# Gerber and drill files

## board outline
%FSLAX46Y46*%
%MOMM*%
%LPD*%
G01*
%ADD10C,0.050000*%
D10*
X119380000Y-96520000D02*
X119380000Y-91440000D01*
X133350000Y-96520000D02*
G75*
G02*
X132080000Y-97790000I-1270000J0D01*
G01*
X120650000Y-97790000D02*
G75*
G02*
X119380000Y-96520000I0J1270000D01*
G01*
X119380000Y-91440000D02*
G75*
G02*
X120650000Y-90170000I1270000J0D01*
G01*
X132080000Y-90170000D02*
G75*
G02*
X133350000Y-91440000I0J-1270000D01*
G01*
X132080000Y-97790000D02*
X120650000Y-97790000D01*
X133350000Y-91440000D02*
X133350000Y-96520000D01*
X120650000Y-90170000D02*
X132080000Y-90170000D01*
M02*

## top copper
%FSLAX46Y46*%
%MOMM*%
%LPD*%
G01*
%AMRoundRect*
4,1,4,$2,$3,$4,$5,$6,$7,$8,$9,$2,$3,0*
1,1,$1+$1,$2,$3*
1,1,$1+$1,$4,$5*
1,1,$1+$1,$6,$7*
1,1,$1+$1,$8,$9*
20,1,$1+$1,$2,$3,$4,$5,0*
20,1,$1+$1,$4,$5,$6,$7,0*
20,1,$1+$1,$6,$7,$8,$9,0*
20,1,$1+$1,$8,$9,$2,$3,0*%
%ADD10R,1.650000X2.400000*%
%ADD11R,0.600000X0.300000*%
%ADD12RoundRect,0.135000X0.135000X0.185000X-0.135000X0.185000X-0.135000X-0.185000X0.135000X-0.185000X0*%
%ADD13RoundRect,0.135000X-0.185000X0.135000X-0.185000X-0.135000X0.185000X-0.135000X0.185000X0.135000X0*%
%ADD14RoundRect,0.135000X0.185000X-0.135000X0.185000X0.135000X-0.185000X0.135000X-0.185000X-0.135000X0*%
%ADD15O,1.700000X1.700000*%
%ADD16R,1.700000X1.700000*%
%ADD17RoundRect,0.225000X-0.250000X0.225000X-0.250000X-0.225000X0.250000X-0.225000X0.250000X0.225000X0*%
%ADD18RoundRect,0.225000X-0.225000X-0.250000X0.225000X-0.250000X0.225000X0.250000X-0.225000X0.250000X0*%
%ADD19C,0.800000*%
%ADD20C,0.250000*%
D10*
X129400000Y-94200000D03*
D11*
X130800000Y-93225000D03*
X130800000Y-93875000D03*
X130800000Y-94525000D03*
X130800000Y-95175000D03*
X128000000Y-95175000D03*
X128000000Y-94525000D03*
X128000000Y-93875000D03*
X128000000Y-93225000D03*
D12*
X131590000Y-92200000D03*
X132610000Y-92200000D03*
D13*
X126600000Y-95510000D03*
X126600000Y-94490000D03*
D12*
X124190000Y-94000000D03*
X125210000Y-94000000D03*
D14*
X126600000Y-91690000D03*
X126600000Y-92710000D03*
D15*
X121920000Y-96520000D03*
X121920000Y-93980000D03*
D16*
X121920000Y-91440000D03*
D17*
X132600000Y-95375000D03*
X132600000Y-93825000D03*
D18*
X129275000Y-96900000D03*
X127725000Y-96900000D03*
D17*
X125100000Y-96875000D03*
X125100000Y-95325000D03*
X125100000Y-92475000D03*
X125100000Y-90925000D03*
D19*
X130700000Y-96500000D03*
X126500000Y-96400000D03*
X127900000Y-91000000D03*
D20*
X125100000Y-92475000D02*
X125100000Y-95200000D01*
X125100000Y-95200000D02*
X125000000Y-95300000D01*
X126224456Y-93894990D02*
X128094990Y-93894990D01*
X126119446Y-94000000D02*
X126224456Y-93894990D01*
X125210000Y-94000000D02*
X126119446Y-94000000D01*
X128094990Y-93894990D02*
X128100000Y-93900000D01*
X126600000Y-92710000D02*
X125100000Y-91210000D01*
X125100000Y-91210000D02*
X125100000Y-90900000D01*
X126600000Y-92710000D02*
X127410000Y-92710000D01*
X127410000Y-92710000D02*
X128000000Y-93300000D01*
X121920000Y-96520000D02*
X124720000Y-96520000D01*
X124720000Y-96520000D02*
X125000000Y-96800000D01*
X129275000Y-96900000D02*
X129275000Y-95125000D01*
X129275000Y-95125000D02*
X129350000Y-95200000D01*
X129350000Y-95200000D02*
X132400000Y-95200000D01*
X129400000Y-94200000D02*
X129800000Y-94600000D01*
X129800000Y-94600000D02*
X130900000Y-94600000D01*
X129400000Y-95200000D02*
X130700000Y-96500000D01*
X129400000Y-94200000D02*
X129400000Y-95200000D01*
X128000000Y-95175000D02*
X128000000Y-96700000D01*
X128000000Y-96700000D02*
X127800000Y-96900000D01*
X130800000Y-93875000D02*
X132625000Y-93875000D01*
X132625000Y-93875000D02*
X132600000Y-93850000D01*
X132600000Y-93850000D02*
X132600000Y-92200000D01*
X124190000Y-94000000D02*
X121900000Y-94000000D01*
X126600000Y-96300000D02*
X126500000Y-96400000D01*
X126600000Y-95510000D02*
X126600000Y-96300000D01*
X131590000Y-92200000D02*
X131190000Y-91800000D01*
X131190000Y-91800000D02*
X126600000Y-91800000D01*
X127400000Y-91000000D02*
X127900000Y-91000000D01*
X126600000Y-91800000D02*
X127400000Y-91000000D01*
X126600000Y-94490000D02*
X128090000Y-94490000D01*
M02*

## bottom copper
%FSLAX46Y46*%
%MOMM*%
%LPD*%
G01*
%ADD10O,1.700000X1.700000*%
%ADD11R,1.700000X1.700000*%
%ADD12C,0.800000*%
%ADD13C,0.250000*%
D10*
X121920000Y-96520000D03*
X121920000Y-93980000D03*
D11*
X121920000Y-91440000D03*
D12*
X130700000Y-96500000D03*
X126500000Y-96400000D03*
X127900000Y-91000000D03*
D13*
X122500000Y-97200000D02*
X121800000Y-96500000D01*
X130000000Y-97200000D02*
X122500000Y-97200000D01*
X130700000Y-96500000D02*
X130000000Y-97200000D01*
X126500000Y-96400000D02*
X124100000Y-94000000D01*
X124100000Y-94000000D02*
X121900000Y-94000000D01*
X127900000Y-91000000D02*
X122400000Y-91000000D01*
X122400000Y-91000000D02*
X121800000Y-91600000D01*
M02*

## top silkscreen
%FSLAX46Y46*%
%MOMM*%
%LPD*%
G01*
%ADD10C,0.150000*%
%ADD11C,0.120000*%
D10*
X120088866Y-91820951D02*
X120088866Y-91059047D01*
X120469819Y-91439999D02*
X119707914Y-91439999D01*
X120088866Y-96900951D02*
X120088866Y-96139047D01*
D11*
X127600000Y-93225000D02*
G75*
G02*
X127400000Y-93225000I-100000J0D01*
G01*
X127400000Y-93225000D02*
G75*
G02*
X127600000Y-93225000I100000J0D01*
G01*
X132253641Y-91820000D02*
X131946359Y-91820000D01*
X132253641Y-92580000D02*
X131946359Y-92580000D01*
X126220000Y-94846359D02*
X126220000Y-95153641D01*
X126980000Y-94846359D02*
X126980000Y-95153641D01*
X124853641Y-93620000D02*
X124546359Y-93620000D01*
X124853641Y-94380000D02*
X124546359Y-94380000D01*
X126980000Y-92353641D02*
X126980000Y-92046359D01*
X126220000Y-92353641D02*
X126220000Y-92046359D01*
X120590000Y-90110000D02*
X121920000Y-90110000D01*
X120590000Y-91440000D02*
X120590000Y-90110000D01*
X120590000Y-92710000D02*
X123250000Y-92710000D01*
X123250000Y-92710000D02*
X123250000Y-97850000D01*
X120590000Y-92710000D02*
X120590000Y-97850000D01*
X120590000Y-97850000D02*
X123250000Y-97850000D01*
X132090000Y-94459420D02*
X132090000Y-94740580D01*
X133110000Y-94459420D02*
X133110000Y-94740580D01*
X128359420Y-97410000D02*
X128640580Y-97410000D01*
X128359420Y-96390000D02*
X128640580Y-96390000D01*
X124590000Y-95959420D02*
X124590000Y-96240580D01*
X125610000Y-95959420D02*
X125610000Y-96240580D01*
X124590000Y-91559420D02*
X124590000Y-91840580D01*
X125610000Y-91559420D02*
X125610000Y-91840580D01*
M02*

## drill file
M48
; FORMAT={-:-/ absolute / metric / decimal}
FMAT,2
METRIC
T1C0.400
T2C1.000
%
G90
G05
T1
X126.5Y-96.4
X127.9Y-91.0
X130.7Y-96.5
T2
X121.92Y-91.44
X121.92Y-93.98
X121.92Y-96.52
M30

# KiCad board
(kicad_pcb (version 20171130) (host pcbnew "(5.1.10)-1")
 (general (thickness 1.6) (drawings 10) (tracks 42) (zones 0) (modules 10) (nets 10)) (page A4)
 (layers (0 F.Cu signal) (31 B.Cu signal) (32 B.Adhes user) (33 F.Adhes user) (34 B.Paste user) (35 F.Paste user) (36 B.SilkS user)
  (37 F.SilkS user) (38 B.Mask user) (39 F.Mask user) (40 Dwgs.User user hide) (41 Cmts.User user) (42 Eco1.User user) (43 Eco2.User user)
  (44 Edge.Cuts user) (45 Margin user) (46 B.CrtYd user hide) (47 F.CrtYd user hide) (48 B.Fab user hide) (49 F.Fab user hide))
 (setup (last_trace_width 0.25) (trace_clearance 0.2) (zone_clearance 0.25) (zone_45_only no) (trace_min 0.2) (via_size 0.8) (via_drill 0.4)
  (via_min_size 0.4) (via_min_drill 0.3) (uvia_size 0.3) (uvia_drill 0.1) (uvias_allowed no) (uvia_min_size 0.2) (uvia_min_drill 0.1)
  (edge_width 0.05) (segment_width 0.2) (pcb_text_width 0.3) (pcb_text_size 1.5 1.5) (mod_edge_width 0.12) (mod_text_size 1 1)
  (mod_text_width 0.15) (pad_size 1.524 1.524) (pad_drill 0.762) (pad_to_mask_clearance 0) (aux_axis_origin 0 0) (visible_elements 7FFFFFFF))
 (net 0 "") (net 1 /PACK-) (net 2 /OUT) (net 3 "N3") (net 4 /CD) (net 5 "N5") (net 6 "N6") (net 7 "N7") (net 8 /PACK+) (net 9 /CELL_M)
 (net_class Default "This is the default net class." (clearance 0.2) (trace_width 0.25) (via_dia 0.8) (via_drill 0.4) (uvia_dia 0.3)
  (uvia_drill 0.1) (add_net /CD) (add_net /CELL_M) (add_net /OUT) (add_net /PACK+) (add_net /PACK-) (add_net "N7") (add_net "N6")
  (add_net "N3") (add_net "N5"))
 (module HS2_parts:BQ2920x (layer F.Cu) (at 129.4 94.2)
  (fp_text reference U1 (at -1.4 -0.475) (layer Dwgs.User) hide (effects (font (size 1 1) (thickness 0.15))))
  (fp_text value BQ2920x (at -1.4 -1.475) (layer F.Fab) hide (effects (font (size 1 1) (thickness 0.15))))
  (fp_circle (center -1.9 -0.975) (end -1.8 -0.975) (layer F.SilkS) (width 0.12))
  (pad 5 smd rect (at 0 0) (size 1.65 2.4) (layers F.Cu F.Paste F.Mask) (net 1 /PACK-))
  (pad 8 smd rect (at 1.4 -0.975) (size 0.6 0.3) (layers F.Cu F.Paste F.Mask) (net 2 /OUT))
  (pad 7 smd rect (at 1.4 -0.325) (size 0.6 0.3) (layers F.Cu F.Paste F.Mask) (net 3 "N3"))
  (pad 6 smd rect (at 1.4 0.325) (size 0.6 0.3) (layers F.Cu F.Paste F.Mask) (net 1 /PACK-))
  (pad 5 smd rect (at 1.4 0.975) (size 0.6 0.3) (layers F.Cu F.Paste F.Mask) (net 1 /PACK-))
  (pad 4 smd rect (at -1.4 0.975) (size 0.6 0.3) (layers F.Cu F.Paste F.Mask) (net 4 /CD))
  (pad 3 smd rect (at -1.4 0.325) (size 0.6 0.3) (layers F.Cu F.Paste F.Mask) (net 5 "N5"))
  (pad 2 smd rect (at -1.4 -0.325) (size 0.6 0.3) (layers F.Cu F.Paste F.Mask) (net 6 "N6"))
  (pad 1 smd rect (at -1.4 -0.975) (size 0.6 0.3) (layers F.Cu F.Paste F.Mask) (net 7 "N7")))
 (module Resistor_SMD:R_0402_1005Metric (layer F.Cu) (at 132.1 92.2 180)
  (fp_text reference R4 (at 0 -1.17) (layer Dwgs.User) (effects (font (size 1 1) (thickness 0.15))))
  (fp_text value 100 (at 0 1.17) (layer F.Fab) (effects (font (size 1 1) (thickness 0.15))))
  (fp_line (start -0.153641 0.38) (end 0.153641 0.38) (layer F.SilkS) (width 0.12))
  (fp_line (start -0.153641 -0.38) (end 0.153641 -0.38) (layer F.SilkS) (width 0.12))
  (pad 2 smd roundrect (at 0.51 0 180) (size 0.54 0.64) (layers F.Cu F.Paste F.Mask) (roundrect_rratio 0.25) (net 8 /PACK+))
  (pad 1 smd roundrect (at -0.51 0 180) (size 0.54 0.64) (layers F.Cu F.Paste F.Mask) (roundrect_rratio 0.25) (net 3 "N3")))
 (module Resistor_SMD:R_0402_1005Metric (layer F.Cu) (at 126.6 95 270)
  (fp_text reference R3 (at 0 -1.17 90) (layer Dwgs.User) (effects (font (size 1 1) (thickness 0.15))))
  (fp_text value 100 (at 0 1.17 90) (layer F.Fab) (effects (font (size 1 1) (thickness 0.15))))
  (fp_line (start -0.153641 0.38) (end 0.153641 0.38) (layer F.SilkS) (width 0.12))
  (fp_line (start -0.153641 -0.38) (end 0.153641 -0.38) (layer F.SilkS) (width 0.12))
  (pad 2 smd roundrect (at 0.51 0 270) (size 0.54 0.64) (layers F.Cu F.Paste F.Mask) (roundrect_rratio 0.25) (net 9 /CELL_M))
  (pad 1 smd roundrect (at -0.51 0 270) (size 0.54 0.64) (layers F.Cu F.Paste F.Mask) (roundrect_rratio 0.25) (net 5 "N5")))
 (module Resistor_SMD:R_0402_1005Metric (layer F.Cu) (at 124.7 94 180)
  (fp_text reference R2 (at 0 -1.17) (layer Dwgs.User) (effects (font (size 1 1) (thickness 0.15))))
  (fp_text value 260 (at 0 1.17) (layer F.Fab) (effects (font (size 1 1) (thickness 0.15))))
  (fp_line (start -0.153641 0.38) (end 0.153641 0.38) (layer F.SilkS) (width 0.12))
  (fp_line (start -0.153641 -0.38) (end 0.153641 -0.38) (layer F.SilkS) (width 0.12))
  (pad 2 smd roundrect (at 0.51 0 180) (size 0.54 0.64) (layers F.Cu F.Paste F.Mask) (roundrect_rratio 0.25) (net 9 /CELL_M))
  (pad 1 smd roundrect (at -0.51 0 180) (size 0.54 0.64) (layers F.Cu F.Paste F.Mask) (roundrect_rratio 0.25) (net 6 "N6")))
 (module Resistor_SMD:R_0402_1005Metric (layer F.Cu) (at 126.6 92.2 90)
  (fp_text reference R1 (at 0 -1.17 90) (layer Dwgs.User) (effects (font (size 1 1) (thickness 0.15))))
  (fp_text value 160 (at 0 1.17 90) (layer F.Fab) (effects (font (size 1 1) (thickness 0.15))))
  (fp_line (start -0.153641 0.38) (end 0.153641 0.38) (layer F.SilkS) (width 0.12))
  (fp_line (start -0.153641 -0.38) (end 0.153641 -0.38) (layer F.SilkS) (width 0.12))
  (pad 2 smd roundrect (at 0.51 0 90) (size 0.54 0.64) (layers F.Cu F.Paste F.Mask) (roundrect_rratio 0.25) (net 8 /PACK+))
  (pad 1 smd roundrect (at -0.51 0 90) (size 0.54 0.64) (layers F.Cu F.Paste F.Mask) (roundrect_rratio 0.25) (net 7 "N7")))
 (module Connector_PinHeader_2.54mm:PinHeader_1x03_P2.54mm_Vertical (layer F.Cu) (at 121.92 91.44)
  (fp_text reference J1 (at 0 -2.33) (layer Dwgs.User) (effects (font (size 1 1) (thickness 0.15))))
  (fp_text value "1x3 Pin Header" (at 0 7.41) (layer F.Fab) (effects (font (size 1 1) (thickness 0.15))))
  (fp_line (start -1.33 -1.33) (end 0 -1.33) (layer F.SilkS) (width 0.12))
  (fp_line (start -1.33 0) (end -1.33 -1.33) (layer F.SilkS) (width 0.12))
  (fp_line (start -1.33 1.27) (end 1.33 1.27) (layer F.SilkS) (width 0.12))
  (fp_line (start 1.33 1.27) (end 1.33 6.41) (layer F.SilkS) (width 0.12))
  (fp_line (start -1.33 1.27) (end -1.33 6.41) (layer F.SilkS) (width 0.12))
  (fp_line (start -1.33 6.41) (end 1.33 6.41) (layer F.SilkS) (width 0.12))
  (pad 3 thru_hole oval (at 0 5.08) (size 1.7 1.7) (drill 1) (layers *.Cu *.Mask) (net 1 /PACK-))
  (pad 2 thru_hole oval (at 0 2.54) (size 1.7 1.7) (drill 1) (layers *.Cu *.Mask) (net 9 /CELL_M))
  (pad 1 thru_hole rect (at 0 0) (size 1.7 1.7) (drill 1) (layers *.Cu *.Mask) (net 8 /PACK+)))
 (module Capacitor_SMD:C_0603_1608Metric (layer F.Cu) (at 132.6 94.6 270)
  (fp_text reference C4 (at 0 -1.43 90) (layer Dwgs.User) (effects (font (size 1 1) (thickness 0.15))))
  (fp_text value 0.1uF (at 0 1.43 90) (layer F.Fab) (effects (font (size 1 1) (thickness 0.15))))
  (fp_line (start -0.14058 0.51) (end 0.14058 0.51) (layer F.SilkS) (width 0.12))
  (fp_line (start -0.14058 -0.51) (end 0.14058 -0.51) (layer F.SilkS) (width 0.12))
  (pad 2 smd roundrect (at 0.775 0 270) (size 0.9 0.95) (layers F.Cu F.Paste F.Mask) (roundrect_rratio 0.25) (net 1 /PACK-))
  (pad 1 smd roundrect (at -0.775 0 270) (size 0.9 0.95) (layers F.Cu F.Paste F.Mask) (roundrect_rratio 0.25) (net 3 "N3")))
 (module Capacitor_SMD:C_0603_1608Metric (layer F.Cu) (at 128.5 96.9)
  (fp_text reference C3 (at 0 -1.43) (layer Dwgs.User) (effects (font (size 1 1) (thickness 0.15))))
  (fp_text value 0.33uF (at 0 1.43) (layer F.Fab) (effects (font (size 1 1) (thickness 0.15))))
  (fp_line (start -0.14058 0.51) (end 0.14058 0.51) (layer F.SilkS) (width 0.12))
  (fp_line (start -0.14058 -0.51) (end 0.14058 -0.51) (layer F.SilkS) (width 0.12))
  (pad 2 smd roundrect (at 0.775 0) (size 0.9 0.95) (layers F.Cu F.Paste F.Mask) (roundrect_rratio 0.25) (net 1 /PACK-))
  (pad 1 smd roundrect (at -0.775 0) (size 0.9 0.95) (layers F.Cu F.Paste F.Mask) (roundrect_rratio 0.25) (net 4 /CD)))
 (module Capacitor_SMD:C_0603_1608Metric (layer F.Cu) (at 125.1 96.1 270)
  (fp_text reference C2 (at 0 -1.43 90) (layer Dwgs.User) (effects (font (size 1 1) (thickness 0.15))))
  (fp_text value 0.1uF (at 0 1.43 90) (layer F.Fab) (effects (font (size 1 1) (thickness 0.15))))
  (fp_line (start -0.14058 0.51) (end 0.14058 0.51) (layer F.SilkS) (width 0.12))
  (fp_line (start -0.14058 -0.51) (end 0.14058 -0.51) (layer F.SilkS) (width 0.12))
  (pad 2 smd roundrect (at 0.775 0 270) (size 0.9 0.95) (layers F.Cu F.Paste F.Mask) (roundrect_rratio 0.25) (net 1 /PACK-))
  (pad 1 smd roundrect (at -0.775 0 270) (size 0.9 0.95) (layers F.Cu F.Paste F.Mask) (roundrect_rratio 0.25) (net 6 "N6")))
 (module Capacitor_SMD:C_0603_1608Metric (layer F.Cu) (at 125.1 91.7 270)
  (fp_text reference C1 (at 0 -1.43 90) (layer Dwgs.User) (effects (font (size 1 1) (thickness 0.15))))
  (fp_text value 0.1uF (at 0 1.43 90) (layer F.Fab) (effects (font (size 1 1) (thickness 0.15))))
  (fp_line (start -0.14058 0.51) (end 0.14058 0.51) (layer F.SilkS) (width 0.12))
  (fp_line (start -0.14058 -0.51) (end 0.14058 -0.51) (layer F.SilkS) (width 0.12))
  (pad 2 smd roundrect (at 0.775 0 270) (size 0.9 0.95) (layers F.Cu F.Paste F.Mask) (roundrect_rratio 0.25) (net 6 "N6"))
  (pad 1 smd roundrect (at -0.775 0 270) (size 0.9 0.95) (layers F.Cu F.Paste F.Mask) (roundrect_rratio 0.25) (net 7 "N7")))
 (gr_line (start 119.38 96.52) (end 119.38 91.44) (layer Edge.Cuts) (width 0.05))
 (gr_arc (start 132.08 96.52) (end 132.08 97.79) (angle -90) (layer Edge.Cuts) (width 0.05))
 (gr_arc (start 120.65 96.52) (end 119.38 96.52) (angle -90) (layer Edge.Cuts) (width 0.05))
 (gr_arc (start 120.65 91.44) (end 120.65 90.17) (angle -90) (layer Edge.Cuts) (width 0.05))
 (gr_arc (start 132.08 91.44) (end 133.35 91.44) (angle -90) (layer Edge.Cuts) (width 0.05))
 (gr_line (start 132.08 97.79) (end 120.65 97.79) (layer Edge.Cuts) (width 0.05))
 (gr_line (start 133.35 91.44) (end 133.35 96.52) (layer Edge.Cuts) (width 0.05))
 (gr_line (start 120.65 90.17) (end 132.08 90.17) (layer Edge.Cuts) (width 0.05))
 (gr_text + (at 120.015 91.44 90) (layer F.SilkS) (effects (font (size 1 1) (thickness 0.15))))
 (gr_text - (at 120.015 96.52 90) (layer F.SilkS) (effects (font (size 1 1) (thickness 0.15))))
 (segment (start 125.1 92.475) (end 125.1 95.2) (width 0.25) (layer F.Cu) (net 6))
 (segment (start 125.1 95.2) (end 125 95.3) (width 0.25) (layer F.Cu) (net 6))
 (segment (start 126.224456 93.89499) (end 128.09499 93.89499) (width 0.25) (layer F.Cu) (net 6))
 (segment (start 126.119446 94) (end 126.224456 93.89499) (width 0.25) (layer F.Cu) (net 6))
 (segment (start 125.21 94) (end 126.119446 94) (width 0.25) (layer F.Cu) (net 6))
 (segment (start 128.09499 93.89499) (end 128.1 93.9) (width 0.25) (layer F.Cu) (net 6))
 (segment (start 126.6 92.71) (end 125.1 91.21) (width 0.25) (layer F.Cu) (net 7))
 (segment (start 125.1 91.21) (end 125.1 90.9) (width 0.25) (layer F.Cu) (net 7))
 (segment (start 126.6 92.71) (end 127.41 92.71) (width 0.25) (layer F.Cu) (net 7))
 (segment (start 127.41 92.71) (end 128 93.3) (width 0.25) (layer F.Cu) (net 7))
 (segment (start 121.92 96.52) (end 124.72 96.52) (width 0.25) (layer F.Cu) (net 1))
 (segment (start 124.72 96.52) (end 125 96.8) (width 0.25) (layer F.Cu) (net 1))
 (segment (start 129.275 96.9) (end 129.275 95.125) (width 0.25) (layer F.Cu) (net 1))
 (segment (start 129.275 95.125) (end 129.35 95.2) (width 0.25) (layer F.Cu) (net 1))
 (segment (start 129.35 95.2) (end 132.4 95.2) (width 0.25) (layer F.Cu) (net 1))
 (segment (start 129.4 94.2) (end 129.8 94.6) (width 0.25) (layer F.Cu) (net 1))
 (segment (start 129.8 94.6) (end 130.9 94.6) (width 0.25) (layer F.Cu) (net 1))
 (via (at 130.7 96.5) (size 0.8) (drill 0.4) (layers F.Cu B.Cu) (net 1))
 (segment (start 129.4 95.2) (end 130.7 96.5) (width 0.25) (layer F.Cu) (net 1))
 (segment (start 129.4 94.2) (end 129.4 95.2) (width 0.25) (layer F.Cu) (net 1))
 (segment (start 122.5 97.2) (end 121.8 96.5) (width 0.25) (layer B.Cu) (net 1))
 (segment (start 130 97.2) (end 122.5 97.2) (width 0.25) (layer B.Cu) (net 1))
 (segment (start 130.7 96.5) (end 130 97.2) (width 0.25) (layer B.Cu) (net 1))
 (segment (start 128 95.175) (end 128 96.7) (width 0.25) (layer F.Cu) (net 4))
 (segment (start 128 96.7) (end 127.8 96.9) (width 0.25) (layer F.Cu) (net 4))
 (segment (start 130.8 93.875) (end 132.625 93.875) (width 0.25) (layer F.Cu) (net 3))
 (segment (start 132.625 93.875) (end 132.6 93.85) (width 0.25) (layer F.Cu) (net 3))
 (segment (start 132.6 93.85) (end 132.6 92.2) (width 0.25) (layer F.Cu) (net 3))
 (segment (start 124.19 94) (end 121.9 94) (width 0.25) (layer F.Cu) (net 9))
 (via (at 126.5 96.4) (size 0.8) (drill 0.4) (layers F.Cu B.Cu) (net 9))
 (segment (start 126.6 96.3) (end 126.5 96.4) (width 0.25) (layer F.Cu) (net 9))
 (segment (start 126.6 95.51) (end 126.6 96.3) (width 0.25) (layer F.Cu) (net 9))
 (segment (start 126.5 96.4) (end 124.1 94) (width 0.25) (layer B.Cu) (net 9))
 (segment (start 124.1 94) (end 121.9 94) (width 0.25) (layer B.Cu) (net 9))
 (segment (start 131.59 92.2) (end 131.19 91.8) (width 0.25) (layer F.Cu) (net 8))
 (segment (start 131.19 91.8) (end 126.6 91.8) (width 0.25) (layer F.Cu) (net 8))
 (segment (start 127.4 91) (end 127.9 91) (width 0.25) (layer F.Cu) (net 8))
 (via (at 127.9 91) (size 0.8) (drill 0.4) (layers F.Cu B.Cu) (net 8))
 (segment (start 126.6 91.8) (end 127.4 91) (width 0.25) (layer F.Cu) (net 8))
 (segment (start 127.9 91) (end 122.4 91) (width 0.25) (layer B.Cu) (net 8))
 (segment (start 122.4 91) (end 121.8 91.6) (width 0.25) (layer B.Cu) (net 8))
 (segment (start 126.6 94.49) (end 128.09 94.49) (width 0.25) (layer F.Cu) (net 5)))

